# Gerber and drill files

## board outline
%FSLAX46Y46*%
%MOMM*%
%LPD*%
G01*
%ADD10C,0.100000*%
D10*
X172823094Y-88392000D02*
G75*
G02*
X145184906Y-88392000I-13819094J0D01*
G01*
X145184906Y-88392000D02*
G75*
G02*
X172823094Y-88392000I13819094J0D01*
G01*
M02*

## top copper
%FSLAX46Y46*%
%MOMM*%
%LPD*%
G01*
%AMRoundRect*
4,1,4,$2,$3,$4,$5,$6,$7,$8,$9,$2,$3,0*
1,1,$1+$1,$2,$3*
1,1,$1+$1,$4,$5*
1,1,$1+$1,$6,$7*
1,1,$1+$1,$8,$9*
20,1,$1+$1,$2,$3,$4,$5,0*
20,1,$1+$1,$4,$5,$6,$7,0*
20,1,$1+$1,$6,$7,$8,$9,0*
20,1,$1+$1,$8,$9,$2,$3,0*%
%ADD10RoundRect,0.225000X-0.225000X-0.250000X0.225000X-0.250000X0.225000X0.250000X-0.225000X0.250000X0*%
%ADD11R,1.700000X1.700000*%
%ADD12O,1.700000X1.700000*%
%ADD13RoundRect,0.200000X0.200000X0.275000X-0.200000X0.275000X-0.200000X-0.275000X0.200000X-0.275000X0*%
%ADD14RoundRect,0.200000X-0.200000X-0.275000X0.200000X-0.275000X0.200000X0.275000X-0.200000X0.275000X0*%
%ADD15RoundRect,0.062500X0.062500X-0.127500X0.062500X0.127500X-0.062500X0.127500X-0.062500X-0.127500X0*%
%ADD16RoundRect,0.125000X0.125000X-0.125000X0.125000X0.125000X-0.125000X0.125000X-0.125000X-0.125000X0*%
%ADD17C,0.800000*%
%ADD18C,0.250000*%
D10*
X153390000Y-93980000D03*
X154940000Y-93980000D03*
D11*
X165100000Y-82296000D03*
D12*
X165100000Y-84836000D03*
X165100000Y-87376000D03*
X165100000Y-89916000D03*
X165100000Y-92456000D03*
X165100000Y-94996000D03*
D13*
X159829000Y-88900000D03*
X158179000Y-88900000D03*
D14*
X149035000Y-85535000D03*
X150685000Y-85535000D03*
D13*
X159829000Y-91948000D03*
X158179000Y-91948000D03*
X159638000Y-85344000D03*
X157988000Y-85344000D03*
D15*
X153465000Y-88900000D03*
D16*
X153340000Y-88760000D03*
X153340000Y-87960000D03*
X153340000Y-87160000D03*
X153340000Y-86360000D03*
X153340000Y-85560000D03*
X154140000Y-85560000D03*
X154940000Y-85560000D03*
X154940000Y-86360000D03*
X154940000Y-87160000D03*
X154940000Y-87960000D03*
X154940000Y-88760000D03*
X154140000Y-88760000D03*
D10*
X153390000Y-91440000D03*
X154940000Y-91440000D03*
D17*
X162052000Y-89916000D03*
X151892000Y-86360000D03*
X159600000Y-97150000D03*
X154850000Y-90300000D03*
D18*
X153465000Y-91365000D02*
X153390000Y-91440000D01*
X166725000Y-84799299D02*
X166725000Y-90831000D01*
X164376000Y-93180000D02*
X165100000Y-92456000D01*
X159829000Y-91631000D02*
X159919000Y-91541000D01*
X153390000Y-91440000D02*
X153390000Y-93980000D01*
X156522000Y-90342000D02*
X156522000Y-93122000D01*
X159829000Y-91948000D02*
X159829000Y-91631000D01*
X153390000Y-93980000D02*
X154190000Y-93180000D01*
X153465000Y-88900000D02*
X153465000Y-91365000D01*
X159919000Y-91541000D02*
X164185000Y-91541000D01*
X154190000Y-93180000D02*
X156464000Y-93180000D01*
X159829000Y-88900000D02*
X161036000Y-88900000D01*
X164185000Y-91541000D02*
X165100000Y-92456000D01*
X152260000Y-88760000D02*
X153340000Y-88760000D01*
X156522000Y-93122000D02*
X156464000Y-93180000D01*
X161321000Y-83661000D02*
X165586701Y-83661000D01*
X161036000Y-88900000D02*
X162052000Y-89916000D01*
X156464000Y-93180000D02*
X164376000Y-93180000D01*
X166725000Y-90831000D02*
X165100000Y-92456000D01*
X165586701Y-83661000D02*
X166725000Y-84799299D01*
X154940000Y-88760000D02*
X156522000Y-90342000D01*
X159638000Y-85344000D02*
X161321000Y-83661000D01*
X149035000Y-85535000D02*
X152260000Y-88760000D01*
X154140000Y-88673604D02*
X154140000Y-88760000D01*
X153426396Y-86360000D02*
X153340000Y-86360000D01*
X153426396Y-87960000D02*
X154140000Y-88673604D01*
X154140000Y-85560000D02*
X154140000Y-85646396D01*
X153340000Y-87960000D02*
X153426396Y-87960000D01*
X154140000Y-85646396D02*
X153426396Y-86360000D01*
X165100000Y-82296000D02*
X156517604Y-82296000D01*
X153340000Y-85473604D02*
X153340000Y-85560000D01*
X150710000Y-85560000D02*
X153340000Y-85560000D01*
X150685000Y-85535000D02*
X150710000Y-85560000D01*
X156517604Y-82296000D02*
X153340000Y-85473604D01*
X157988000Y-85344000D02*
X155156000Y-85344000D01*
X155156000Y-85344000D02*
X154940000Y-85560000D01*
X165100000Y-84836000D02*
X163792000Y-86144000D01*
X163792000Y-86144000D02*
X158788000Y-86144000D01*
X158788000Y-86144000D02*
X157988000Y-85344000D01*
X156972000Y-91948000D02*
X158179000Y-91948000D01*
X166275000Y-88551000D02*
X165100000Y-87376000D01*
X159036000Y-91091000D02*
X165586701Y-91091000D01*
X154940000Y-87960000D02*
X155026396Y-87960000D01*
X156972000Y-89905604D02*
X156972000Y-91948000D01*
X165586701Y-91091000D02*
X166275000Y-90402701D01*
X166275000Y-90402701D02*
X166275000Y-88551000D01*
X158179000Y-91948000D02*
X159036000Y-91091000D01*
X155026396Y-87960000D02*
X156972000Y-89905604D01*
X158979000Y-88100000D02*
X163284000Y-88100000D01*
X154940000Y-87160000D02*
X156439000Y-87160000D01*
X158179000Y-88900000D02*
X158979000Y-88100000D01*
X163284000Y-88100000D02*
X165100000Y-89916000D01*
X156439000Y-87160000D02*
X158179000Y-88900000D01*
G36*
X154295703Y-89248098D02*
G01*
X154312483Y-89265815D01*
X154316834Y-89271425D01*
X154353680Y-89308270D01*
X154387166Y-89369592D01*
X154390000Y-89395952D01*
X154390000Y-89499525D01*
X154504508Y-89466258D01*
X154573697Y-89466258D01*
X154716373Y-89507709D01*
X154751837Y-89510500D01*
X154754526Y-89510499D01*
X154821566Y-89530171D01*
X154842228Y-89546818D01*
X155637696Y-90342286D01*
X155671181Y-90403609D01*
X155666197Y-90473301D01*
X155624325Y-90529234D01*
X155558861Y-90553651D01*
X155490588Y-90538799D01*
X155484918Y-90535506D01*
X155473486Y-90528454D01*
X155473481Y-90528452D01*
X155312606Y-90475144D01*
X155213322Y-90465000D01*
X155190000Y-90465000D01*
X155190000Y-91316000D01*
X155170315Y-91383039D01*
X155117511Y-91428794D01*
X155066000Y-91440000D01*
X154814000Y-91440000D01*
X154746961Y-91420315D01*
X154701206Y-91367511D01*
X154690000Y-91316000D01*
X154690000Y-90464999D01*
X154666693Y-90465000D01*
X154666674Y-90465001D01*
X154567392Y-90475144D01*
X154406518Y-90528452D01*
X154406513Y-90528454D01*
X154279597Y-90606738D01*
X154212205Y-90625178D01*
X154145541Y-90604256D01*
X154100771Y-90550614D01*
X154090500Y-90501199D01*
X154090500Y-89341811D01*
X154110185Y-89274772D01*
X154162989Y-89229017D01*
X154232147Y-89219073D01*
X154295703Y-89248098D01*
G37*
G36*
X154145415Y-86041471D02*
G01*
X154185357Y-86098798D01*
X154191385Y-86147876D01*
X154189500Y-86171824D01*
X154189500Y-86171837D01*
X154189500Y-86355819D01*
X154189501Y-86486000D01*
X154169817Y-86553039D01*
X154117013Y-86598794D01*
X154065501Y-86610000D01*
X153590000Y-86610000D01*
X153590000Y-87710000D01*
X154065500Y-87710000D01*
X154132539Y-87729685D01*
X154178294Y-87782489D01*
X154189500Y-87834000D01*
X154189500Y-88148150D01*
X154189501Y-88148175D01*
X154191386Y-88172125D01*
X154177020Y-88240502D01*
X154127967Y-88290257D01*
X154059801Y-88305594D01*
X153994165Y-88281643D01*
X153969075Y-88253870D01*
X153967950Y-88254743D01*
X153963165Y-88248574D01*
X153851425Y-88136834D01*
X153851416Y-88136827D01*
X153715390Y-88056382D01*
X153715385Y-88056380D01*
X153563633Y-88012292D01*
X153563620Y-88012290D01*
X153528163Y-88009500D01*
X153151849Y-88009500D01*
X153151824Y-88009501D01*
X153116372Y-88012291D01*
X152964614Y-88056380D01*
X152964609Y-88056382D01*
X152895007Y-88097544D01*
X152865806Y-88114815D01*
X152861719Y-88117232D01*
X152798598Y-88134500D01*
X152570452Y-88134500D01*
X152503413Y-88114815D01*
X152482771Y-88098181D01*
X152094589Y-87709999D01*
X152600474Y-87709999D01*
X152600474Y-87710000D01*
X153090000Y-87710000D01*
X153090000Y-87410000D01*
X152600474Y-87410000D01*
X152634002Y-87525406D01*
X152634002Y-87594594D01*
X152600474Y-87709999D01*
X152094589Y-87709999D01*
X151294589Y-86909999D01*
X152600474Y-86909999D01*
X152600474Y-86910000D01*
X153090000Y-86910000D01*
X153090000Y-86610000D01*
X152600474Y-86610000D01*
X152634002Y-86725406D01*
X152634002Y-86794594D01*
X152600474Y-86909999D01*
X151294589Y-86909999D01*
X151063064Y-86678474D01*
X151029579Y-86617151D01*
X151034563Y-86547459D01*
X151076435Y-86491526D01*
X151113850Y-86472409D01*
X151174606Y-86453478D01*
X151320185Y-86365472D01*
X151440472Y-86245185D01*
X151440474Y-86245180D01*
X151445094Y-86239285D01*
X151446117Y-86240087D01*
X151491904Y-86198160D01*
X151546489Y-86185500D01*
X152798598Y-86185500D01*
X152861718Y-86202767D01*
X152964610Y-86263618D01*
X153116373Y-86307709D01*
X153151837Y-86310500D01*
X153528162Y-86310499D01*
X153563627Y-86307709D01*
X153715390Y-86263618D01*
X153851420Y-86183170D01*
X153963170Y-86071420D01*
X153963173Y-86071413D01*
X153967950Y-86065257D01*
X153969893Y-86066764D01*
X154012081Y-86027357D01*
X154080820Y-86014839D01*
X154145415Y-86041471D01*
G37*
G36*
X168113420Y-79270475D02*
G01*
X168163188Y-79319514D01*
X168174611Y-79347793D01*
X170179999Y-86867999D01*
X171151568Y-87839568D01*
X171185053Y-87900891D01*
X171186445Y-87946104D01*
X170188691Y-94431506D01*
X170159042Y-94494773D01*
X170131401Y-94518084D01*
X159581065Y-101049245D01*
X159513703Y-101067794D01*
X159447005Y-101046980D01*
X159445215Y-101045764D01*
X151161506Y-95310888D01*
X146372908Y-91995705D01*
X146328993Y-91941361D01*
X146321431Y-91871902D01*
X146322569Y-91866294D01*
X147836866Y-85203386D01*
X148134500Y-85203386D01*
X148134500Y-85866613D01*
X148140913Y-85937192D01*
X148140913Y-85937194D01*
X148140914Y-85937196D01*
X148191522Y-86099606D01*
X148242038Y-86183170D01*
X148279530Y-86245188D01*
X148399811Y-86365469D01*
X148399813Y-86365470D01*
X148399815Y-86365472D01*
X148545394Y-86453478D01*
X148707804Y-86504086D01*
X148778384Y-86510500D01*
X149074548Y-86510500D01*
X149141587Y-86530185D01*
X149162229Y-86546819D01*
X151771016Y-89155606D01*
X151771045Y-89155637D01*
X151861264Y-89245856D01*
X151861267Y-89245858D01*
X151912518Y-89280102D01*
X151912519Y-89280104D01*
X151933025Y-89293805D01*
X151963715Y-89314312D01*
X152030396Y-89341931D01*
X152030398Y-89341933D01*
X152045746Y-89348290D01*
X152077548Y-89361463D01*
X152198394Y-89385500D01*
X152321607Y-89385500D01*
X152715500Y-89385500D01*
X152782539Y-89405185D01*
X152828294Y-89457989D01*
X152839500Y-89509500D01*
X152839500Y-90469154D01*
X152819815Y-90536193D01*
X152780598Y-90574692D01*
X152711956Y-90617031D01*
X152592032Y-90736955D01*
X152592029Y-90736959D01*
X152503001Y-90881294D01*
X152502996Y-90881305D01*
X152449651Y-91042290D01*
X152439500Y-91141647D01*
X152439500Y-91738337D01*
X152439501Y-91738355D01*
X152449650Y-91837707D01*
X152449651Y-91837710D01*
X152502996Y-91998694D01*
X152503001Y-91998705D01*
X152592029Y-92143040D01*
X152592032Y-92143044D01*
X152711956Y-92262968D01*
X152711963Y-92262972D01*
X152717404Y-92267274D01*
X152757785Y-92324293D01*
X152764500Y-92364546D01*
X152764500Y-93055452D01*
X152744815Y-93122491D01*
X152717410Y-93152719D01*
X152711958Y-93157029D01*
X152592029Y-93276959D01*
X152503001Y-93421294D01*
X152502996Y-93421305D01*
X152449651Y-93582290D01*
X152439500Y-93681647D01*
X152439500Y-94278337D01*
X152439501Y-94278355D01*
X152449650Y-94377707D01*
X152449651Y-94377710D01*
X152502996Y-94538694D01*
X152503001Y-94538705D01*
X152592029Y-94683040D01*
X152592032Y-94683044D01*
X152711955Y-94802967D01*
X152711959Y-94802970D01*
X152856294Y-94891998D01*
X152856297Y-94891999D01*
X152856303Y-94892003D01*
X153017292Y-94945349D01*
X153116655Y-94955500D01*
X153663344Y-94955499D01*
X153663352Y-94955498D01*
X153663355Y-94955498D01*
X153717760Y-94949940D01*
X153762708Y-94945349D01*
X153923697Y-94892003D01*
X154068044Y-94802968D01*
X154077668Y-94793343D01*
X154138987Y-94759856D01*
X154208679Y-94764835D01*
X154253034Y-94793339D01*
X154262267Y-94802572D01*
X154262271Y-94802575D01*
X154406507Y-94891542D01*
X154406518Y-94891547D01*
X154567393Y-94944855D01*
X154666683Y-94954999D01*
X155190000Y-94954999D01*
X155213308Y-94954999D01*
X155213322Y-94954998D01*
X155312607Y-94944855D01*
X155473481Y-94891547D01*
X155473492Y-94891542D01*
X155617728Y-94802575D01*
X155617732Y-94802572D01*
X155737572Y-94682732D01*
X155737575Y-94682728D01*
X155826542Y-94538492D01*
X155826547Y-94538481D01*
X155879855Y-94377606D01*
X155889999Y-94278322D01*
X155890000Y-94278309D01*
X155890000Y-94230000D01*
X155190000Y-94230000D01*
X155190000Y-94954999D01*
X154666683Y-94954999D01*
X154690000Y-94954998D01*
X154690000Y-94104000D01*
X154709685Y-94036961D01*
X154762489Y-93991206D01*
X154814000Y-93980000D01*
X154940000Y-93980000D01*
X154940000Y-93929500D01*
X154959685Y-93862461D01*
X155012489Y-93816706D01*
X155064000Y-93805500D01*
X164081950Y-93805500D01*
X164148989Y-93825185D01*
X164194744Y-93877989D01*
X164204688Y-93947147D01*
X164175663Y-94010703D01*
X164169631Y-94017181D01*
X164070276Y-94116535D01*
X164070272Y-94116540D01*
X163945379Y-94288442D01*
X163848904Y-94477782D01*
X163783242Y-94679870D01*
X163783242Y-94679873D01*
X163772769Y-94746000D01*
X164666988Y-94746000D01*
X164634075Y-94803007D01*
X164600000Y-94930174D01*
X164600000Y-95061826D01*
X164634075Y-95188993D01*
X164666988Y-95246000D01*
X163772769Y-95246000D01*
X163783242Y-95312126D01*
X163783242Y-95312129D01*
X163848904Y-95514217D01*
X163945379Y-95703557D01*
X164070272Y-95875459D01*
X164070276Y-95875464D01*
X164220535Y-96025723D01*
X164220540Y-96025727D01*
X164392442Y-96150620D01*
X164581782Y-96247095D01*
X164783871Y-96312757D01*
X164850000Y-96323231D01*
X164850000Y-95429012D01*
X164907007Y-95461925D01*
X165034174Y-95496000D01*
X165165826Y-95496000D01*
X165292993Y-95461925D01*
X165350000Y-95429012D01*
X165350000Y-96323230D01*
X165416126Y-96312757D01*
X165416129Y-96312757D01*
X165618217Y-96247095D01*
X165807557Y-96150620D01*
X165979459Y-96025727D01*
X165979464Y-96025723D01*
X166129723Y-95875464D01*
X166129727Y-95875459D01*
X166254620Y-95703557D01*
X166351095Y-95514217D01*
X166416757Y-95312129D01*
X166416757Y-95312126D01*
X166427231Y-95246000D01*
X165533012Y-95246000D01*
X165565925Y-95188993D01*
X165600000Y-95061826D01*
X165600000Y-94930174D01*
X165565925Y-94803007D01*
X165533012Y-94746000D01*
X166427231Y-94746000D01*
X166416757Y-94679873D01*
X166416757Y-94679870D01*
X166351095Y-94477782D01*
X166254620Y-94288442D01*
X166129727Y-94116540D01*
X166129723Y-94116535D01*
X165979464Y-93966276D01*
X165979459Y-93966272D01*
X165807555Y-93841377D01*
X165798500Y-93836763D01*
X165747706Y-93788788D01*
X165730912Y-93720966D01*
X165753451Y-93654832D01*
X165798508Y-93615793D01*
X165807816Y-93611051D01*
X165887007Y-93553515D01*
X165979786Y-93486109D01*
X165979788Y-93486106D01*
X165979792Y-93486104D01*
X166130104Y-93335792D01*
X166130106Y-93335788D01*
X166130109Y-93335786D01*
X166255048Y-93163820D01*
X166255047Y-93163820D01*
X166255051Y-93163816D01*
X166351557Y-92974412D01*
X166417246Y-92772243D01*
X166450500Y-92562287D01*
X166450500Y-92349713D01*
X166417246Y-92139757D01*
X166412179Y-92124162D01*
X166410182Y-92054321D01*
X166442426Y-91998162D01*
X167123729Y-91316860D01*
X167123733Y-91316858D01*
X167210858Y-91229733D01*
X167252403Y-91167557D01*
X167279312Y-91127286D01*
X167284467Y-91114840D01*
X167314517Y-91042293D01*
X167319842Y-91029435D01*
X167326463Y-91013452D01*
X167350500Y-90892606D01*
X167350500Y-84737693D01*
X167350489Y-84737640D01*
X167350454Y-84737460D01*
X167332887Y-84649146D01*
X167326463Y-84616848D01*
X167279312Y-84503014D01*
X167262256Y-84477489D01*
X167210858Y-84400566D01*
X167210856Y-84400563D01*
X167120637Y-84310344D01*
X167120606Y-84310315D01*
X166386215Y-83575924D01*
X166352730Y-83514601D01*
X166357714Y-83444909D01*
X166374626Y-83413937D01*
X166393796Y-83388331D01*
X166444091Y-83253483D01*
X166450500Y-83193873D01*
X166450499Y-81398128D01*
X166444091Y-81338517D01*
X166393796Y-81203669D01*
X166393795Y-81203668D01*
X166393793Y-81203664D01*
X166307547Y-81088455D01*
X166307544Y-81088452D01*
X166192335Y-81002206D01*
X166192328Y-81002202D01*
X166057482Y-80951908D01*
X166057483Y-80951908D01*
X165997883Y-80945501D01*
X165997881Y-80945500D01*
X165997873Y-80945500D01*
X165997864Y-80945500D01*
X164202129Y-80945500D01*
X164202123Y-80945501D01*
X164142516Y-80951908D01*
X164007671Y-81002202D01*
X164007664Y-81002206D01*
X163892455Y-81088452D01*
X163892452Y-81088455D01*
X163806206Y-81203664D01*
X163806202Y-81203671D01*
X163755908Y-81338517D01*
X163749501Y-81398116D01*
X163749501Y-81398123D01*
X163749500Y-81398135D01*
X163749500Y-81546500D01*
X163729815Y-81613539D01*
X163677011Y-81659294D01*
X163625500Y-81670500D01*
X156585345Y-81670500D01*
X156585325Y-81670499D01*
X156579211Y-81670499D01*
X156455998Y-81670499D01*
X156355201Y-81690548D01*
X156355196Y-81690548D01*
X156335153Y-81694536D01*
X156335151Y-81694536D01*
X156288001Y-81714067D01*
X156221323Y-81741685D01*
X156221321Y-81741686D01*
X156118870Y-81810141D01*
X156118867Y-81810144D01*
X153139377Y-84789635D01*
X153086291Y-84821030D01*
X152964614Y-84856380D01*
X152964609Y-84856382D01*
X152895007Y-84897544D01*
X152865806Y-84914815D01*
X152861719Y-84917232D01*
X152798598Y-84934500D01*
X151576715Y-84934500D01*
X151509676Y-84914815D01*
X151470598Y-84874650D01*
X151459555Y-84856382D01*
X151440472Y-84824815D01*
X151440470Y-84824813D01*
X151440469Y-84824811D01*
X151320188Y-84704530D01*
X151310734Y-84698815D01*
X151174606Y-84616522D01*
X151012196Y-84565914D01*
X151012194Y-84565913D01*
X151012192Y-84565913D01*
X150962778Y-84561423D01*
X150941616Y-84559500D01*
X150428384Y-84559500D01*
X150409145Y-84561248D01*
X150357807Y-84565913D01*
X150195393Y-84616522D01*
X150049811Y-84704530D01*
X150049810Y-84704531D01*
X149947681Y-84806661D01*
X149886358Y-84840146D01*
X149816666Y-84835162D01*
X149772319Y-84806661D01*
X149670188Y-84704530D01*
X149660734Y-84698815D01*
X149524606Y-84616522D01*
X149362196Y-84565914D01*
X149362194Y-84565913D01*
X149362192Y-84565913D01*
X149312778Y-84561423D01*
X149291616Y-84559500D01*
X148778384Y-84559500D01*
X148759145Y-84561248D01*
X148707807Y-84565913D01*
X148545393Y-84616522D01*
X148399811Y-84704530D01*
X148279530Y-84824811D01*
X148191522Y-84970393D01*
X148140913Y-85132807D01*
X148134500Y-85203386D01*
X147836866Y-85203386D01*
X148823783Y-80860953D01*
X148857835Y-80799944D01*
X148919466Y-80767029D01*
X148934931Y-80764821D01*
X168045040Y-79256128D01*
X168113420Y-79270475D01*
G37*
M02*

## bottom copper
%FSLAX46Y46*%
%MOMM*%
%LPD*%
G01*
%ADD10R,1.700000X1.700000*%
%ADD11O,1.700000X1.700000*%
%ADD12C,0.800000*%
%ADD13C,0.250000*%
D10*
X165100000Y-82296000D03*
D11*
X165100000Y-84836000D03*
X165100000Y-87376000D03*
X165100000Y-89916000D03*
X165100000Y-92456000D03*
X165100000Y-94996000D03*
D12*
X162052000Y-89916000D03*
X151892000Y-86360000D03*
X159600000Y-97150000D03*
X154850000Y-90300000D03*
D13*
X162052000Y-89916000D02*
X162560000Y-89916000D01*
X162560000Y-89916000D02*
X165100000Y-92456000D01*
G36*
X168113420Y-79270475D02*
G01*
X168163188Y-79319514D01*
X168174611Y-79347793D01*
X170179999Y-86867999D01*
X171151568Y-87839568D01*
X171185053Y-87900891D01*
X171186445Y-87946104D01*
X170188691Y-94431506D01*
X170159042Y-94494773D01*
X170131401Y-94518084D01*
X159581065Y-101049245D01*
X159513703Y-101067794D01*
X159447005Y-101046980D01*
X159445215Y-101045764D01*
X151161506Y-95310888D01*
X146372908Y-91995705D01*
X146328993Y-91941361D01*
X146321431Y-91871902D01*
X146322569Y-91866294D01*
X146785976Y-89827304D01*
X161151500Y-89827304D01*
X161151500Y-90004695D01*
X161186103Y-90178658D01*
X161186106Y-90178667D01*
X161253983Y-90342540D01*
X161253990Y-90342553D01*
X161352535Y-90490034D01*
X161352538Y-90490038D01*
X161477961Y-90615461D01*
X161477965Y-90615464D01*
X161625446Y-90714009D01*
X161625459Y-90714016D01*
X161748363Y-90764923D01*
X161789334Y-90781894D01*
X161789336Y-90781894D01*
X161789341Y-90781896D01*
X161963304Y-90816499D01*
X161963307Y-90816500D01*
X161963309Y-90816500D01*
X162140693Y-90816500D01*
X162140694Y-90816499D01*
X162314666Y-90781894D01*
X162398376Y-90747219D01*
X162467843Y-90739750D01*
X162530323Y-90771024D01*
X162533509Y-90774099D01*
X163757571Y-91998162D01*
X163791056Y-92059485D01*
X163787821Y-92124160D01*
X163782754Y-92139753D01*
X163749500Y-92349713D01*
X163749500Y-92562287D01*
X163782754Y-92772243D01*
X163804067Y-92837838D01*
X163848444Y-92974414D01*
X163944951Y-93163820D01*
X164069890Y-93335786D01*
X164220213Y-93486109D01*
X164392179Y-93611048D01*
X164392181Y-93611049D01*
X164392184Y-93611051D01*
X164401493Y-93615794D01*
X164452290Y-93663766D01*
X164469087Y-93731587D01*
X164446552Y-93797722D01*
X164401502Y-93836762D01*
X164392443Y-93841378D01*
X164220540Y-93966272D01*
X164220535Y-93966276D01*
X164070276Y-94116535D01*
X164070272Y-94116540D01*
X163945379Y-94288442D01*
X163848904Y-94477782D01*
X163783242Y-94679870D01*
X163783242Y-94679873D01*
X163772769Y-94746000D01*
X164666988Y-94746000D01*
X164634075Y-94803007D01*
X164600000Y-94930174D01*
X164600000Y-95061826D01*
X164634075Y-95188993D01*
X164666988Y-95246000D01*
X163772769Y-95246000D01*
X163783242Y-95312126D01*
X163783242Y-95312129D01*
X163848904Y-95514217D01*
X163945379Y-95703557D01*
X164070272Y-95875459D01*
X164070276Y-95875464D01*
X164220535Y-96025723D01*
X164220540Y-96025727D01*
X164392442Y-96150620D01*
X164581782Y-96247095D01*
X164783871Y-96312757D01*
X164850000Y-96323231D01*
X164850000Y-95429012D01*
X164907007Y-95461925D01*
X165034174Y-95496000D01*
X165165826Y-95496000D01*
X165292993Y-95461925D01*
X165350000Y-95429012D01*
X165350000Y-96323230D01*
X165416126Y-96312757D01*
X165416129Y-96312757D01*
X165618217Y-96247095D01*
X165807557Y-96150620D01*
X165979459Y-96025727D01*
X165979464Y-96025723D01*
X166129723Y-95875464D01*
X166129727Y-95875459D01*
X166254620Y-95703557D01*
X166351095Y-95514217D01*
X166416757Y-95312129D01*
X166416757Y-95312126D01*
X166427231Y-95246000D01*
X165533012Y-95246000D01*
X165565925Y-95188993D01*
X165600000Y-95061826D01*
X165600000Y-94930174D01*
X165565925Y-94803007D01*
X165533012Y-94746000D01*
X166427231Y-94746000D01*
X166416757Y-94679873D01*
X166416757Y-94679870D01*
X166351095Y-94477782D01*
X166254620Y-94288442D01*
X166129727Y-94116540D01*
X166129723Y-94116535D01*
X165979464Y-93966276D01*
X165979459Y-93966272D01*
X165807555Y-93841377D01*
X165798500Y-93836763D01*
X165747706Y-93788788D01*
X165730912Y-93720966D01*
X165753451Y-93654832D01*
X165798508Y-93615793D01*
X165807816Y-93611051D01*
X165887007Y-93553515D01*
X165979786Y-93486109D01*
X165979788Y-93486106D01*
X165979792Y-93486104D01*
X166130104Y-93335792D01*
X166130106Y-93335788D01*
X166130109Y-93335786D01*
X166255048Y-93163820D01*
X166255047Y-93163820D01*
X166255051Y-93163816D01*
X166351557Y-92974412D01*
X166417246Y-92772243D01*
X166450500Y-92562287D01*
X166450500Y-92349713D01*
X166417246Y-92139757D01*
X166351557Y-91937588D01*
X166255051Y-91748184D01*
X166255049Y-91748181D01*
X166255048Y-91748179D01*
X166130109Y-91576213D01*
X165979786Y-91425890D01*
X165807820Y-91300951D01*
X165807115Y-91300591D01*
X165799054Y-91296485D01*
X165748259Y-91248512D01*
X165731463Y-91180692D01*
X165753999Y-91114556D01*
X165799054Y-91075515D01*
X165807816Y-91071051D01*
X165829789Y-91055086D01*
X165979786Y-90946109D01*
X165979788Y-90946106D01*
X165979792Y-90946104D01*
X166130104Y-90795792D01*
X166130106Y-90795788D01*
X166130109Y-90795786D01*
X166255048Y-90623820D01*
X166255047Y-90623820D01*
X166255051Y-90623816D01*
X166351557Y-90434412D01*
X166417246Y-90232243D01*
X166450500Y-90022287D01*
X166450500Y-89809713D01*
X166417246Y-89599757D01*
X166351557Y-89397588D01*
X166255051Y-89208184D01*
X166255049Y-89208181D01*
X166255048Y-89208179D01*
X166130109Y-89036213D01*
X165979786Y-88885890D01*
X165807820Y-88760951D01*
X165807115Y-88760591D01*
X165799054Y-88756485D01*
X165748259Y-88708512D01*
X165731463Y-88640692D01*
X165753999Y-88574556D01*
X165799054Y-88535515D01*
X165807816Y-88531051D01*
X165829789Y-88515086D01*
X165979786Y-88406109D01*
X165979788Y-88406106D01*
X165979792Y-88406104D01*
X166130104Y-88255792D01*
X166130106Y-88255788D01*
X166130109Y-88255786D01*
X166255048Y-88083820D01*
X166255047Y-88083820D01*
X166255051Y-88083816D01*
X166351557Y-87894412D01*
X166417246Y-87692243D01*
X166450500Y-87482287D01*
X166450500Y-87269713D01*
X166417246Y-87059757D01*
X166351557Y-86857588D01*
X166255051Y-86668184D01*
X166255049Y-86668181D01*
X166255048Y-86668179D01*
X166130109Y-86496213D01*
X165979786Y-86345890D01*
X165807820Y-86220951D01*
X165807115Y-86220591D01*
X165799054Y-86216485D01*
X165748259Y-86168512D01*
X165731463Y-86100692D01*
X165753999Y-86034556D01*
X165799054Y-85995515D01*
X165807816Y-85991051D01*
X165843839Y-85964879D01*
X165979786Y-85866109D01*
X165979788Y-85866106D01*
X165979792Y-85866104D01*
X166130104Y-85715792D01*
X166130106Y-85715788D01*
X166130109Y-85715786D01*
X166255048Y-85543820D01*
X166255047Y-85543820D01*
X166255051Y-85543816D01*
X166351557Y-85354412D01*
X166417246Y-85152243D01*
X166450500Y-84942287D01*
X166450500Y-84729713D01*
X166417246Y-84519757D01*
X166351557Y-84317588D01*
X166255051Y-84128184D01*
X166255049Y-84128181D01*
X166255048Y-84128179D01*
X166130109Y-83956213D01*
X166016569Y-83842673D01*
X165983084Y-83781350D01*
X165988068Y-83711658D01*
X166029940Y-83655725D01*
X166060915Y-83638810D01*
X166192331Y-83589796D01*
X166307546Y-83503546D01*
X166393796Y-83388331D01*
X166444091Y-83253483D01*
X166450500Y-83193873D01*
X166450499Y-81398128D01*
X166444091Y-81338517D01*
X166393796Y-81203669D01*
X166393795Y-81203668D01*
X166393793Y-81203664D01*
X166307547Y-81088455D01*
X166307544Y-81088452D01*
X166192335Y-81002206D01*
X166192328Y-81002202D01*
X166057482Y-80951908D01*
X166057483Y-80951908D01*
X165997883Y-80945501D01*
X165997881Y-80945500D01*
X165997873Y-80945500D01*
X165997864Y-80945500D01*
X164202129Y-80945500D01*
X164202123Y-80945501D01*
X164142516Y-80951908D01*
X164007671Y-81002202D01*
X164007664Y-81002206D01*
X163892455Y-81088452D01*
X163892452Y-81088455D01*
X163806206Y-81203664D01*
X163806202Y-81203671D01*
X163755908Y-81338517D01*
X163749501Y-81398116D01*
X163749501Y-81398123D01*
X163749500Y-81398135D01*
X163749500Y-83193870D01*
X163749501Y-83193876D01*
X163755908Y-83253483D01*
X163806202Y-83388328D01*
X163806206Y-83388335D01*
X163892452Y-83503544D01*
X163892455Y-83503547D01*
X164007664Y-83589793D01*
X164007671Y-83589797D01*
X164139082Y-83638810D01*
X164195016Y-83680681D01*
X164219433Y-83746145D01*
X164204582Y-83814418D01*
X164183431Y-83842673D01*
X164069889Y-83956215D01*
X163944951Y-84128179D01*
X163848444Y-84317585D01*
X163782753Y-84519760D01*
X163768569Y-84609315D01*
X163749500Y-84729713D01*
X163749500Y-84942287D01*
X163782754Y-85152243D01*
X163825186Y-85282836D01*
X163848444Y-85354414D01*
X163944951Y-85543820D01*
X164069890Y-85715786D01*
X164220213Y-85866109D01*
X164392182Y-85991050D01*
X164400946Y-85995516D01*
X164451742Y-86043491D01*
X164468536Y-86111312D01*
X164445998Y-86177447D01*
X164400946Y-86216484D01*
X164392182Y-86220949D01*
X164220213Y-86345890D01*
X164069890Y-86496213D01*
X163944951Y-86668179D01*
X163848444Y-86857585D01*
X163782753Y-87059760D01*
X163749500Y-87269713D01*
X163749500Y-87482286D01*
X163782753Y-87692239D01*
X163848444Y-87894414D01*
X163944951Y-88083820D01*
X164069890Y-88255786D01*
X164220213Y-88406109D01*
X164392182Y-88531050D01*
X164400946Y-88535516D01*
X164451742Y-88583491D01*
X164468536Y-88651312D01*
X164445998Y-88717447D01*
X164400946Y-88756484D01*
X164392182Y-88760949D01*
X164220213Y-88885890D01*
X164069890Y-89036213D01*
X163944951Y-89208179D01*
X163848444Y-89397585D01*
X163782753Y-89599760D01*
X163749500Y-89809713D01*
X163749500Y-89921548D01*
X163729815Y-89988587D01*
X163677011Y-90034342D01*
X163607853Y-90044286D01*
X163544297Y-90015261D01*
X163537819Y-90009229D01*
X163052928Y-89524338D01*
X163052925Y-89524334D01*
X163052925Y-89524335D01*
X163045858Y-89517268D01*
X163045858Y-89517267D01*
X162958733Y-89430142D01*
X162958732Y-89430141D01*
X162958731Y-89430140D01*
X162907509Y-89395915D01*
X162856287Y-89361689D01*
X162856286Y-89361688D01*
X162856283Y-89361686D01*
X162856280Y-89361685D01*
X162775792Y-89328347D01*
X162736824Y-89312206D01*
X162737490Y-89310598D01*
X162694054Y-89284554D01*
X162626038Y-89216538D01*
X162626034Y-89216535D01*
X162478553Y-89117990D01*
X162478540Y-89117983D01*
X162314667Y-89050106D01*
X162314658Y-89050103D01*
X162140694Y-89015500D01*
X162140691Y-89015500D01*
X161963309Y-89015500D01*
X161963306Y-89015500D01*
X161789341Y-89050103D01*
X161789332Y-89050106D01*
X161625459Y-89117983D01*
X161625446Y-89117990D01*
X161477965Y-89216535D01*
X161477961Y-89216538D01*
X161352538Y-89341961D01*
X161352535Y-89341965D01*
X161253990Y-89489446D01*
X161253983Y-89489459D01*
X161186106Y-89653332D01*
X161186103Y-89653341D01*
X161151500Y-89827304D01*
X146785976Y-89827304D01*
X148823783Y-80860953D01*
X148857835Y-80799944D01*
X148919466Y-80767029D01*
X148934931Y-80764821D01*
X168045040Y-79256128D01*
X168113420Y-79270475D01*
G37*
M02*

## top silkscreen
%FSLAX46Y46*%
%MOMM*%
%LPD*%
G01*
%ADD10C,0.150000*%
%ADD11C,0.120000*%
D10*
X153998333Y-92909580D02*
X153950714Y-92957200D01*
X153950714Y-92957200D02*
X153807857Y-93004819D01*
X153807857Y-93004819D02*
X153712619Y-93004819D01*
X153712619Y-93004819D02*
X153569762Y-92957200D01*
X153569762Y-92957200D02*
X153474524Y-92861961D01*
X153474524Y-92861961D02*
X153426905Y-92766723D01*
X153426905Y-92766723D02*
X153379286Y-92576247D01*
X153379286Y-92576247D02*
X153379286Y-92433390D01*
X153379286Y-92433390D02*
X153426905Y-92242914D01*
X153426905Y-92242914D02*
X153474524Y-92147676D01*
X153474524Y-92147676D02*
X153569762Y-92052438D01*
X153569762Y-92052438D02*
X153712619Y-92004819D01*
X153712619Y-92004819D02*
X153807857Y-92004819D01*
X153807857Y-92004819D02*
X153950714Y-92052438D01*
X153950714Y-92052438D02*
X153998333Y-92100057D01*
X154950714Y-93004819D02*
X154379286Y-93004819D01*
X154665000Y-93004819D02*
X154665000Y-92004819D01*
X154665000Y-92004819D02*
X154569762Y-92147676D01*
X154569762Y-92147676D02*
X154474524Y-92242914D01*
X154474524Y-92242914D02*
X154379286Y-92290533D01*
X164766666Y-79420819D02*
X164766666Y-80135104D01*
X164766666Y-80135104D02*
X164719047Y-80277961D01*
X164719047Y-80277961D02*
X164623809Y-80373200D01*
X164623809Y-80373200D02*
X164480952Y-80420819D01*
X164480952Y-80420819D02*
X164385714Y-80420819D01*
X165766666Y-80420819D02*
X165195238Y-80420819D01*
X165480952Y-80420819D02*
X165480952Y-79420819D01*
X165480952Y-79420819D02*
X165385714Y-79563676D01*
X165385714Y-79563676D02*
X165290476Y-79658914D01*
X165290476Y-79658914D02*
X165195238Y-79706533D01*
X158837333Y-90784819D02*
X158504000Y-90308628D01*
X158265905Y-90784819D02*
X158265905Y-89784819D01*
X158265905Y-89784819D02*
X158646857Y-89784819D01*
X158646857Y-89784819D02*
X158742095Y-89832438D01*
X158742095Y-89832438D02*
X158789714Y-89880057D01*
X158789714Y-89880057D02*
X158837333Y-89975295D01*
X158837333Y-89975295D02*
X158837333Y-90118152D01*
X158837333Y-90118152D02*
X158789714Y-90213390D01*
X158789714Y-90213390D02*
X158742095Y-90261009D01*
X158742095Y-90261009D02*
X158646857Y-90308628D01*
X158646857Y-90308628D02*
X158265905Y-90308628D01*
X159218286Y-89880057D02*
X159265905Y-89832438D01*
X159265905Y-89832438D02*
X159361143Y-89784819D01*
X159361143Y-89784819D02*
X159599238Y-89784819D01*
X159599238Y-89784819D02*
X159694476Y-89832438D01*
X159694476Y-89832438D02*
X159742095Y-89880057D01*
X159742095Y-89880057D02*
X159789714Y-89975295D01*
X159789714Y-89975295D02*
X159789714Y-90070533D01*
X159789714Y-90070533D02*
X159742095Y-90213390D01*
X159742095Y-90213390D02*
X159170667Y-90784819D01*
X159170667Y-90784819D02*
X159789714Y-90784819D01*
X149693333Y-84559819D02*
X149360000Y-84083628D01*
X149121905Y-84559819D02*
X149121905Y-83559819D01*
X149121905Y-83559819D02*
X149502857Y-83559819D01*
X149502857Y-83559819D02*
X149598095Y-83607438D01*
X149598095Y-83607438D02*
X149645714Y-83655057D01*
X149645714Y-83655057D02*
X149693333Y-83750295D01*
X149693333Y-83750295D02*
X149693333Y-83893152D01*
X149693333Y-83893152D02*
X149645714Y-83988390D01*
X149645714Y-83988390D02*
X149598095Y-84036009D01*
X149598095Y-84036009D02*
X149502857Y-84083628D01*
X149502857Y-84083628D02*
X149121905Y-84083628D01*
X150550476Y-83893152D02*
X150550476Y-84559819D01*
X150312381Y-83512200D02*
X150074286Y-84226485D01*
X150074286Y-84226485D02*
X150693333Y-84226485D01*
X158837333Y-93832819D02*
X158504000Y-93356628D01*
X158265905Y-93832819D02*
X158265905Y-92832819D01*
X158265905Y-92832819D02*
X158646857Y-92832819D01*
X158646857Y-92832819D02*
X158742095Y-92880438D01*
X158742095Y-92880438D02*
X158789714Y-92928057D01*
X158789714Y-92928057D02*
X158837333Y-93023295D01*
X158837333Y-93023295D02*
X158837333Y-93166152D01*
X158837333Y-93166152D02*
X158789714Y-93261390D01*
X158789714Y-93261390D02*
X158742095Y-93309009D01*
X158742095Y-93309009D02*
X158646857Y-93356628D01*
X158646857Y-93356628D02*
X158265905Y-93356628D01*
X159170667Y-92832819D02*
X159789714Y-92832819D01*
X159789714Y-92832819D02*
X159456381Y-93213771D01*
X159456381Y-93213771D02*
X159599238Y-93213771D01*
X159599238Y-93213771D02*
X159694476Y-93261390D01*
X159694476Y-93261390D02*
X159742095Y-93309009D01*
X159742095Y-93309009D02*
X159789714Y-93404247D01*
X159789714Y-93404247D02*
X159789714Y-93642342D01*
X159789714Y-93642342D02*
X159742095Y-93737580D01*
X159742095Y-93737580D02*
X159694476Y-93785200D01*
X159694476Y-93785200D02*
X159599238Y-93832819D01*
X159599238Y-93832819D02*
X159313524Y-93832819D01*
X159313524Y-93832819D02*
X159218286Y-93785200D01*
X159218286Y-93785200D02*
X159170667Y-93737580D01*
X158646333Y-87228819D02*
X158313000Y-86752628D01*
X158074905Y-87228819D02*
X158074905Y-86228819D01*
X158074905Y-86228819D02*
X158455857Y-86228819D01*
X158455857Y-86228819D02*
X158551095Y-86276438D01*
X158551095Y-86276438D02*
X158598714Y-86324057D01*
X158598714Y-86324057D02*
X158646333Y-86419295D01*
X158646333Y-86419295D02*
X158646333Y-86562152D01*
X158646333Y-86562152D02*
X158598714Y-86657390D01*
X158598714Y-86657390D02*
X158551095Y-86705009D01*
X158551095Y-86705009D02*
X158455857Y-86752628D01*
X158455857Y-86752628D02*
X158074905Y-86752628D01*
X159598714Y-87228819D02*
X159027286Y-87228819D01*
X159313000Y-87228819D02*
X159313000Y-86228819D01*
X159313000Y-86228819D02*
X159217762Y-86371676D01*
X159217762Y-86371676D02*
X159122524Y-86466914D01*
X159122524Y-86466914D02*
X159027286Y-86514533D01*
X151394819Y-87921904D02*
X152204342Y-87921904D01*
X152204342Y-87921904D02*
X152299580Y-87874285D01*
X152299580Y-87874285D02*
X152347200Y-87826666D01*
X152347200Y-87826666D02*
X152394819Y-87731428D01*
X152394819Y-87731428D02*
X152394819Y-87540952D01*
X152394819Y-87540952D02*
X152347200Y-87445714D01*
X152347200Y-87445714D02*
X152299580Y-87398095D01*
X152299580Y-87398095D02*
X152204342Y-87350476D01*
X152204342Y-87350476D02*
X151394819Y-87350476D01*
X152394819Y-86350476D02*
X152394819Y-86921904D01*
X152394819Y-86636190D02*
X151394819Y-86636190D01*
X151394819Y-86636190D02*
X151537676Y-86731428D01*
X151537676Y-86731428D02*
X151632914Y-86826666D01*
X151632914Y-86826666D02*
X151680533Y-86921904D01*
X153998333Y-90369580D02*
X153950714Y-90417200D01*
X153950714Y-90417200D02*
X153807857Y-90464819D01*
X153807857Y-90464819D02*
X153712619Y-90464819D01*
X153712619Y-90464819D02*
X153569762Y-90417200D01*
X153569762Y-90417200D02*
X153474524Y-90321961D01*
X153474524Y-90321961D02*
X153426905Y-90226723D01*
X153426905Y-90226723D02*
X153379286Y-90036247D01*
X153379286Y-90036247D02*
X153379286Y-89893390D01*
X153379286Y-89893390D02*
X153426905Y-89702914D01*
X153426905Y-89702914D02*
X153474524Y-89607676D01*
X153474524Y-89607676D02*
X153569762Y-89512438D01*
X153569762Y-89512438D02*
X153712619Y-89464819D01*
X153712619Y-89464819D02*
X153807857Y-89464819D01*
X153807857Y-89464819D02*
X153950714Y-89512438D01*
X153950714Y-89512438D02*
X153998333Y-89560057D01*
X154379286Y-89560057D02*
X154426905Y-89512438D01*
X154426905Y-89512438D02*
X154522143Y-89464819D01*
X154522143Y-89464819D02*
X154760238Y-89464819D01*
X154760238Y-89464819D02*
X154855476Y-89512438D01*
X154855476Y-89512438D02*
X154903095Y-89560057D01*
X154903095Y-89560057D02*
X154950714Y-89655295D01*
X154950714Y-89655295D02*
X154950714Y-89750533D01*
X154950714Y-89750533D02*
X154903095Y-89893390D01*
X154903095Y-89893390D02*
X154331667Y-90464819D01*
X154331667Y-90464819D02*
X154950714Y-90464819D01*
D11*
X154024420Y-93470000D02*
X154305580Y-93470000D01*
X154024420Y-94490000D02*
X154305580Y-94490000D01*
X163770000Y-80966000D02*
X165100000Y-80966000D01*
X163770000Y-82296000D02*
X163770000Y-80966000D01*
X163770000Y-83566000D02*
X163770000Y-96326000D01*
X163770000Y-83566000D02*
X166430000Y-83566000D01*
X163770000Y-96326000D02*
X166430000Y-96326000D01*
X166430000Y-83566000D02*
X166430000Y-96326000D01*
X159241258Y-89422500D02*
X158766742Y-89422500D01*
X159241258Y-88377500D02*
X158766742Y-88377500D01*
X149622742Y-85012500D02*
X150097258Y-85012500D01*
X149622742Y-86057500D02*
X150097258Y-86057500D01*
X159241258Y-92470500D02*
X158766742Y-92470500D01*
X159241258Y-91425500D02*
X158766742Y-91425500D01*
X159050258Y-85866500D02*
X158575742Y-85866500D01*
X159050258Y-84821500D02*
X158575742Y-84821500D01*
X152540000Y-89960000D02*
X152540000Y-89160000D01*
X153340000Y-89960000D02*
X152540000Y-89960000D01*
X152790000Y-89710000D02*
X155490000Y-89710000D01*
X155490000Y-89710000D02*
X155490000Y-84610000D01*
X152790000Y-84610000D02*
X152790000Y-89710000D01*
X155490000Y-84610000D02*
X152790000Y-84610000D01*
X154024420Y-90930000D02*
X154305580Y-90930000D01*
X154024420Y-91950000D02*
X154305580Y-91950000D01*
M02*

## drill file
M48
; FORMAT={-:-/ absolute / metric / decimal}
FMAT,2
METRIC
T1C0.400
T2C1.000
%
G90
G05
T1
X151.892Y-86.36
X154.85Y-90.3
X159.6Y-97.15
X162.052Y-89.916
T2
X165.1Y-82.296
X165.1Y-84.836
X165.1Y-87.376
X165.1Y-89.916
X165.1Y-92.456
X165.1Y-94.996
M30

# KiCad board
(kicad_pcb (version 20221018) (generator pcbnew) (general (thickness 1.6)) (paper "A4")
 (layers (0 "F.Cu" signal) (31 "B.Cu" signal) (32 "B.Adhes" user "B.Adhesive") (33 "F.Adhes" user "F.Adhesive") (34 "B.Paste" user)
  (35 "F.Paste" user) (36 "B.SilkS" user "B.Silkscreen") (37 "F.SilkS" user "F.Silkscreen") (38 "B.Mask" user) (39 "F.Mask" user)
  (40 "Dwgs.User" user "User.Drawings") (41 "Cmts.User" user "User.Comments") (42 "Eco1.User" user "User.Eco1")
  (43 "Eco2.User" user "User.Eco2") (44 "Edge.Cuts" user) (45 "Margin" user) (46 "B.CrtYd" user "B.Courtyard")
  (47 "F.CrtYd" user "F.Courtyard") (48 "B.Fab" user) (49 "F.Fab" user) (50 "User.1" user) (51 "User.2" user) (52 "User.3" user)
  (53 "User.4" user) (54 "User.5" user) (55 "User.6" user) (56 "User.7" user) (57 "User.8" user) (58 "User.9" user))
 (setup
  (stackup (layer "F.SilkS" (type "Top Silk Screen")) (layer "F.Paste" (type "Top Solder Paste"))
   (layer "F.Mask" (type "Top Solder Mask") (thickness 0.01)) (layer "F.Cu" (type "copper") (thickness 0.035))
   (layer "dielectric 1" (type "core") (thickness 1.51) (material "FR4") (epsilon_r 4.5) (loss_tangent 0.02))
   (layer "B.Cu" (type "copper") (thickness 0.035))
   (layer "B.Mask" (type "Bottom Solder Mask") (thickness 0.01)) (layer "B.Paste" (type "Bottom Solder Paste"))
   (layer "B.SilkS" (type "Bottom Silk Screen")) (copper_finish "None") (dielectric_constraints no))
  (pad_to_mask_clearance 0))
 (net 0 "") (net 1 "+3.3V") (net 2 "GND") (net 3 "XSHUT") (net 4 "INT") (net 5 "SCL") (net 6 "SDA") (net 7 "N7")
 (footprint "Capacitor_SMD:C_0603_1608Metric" (layer "F.Cu") (at 154.165 93.98)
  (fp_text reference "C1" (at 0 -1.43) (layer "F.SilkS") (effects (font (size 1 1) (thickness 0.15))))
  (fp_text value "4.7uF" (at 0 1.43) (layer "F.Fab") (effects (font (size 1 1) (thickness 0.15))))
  (fp_line (start -0.14058 -0.51) (end 0.14058 -0.51) (stroke (width 0.12) (type solid)) (layer "F.SilkS"))
  (fp_line (start -0.14058 0.51) (end 0.14058 0.51) (stroke (width 0.12) (type solid)) (layer "F.SilkS"))
  (pad "1" smd roundrect (at -0.775 0) (size 0.9 0.95) (layers "F.Cu" "F.Paste" "F.Mask") (roundrect_rratio 0.25) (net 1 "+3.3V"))
  (pad "2" smd roundrect (at 0.775 0) (size 0.9 0.95) (layers "F.Cu" "F.Paste" "F.Mask") (roundrect_rratio 0.25) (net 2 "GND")))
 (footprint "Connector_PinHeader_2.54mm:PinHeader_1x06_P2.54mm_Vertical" (layer "F.Cu") (at 165.1 82.296)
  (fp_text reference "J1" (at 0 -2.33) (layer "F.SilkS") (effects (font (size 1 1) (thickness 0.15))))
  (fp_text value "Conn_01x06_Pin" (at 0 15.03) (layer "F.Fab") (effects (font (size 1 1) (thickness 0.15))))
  (fp_line (start -1.33 -1.33) (end 0 -1.33) (stroke (width 0.12) (type solid)) (layer "F.SilkS"))
  (fp_line (start -1.33 0) (end -1.33 -1.33) (stroke (width 0.12) (type solid)) (layer "F.SilkS"))
  (fp_line (start -1.33 1.27) (end -1.33 14.03) (stroke (width 0.12) (type solid)) (layer "F.SilkS"))
  (fp_line (start -1.33 1.27) (end 1.33 1.27) (stroke (width 0.12) (type solid)) (layer "F.SilkS"))
  (fp_line (start -1.33 14.03) (end 1.33 14.03) (stroke (width 0.12) (type solid)) (layer "F.SilkS"))
  (fp_line (start 1.33 1.27) (end 1.33 14.03) (stroke (width 0.12) (type solid)) (layer "F.SilkS"))
  (pad "1" thru_hole rect (at 0 0) (size 1.7 1.7) (drill 1) (layers "*.Cu" "*.Mask") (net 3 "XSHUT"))
  (pad "2" thru_hole oval (at 0 2.54) (size 1.7 1.7) (drill 1) (layers "*.Cu" "*.Mask") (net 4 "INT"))
  (pad "3" thru_hole oval (at 0 5.08) (size 1.7 1.7) (drill 1) (layers "*.Cu" "*.Mask") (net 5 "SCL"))
  (pad "4" thru_hole oval (at 0 7.62) (size 1.7 1.7) (drill 1) (layers "*.Cu" "*.Mask") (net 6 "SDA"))
  (pad "5" thru_hole oval (at 0 10.16) (size 1.7 1.7) (drill 1) (layers "*.Cu" "*.Mask") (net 1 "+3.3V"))
  (pad "6" thru_hole oval (at 0 12.7) (size 1.7 1.7) (drill 1) (layers "*.Cu" "*.Mask") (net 2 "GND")))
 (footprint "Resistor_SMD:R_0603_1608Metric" (layer "F.Cu") (at 159.004 88.9 180)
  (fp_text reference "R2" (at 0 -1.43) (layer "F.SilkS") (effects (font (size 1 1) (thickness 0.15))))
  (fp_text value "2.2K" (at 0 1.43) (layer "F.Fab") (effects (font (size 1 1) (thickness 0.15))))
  (fp_line (start -0.237258 -0.5225) (end 0.237258 -0.5225) (stroke (width 0.12) (type solid)) (layer "F.SilkS"))
  (fp_line (start -0.237258 0.5225) (end 0.237258 0.5225) (stroke (width 0.12) (type solid)) (layer "F.SilkS"))
  (pad "1" smd roundrect (at -0.825 0 180) (size 0.8 0.95) (layers "F.Cu" "F.Paste" "F.Mask") (roundrect_rratio 0.25) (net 1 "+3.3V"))
  (pad "2" smd roundrect (at 0.825 0 180) (size 0.8 0.95) (layers "F.Cu" "F.Paste" "F.Mask") (roundrect_rratio 0.25) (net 6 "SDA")))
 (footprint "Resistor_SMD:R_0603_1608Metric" (layer "F.Cu") (at 149.86 85.535)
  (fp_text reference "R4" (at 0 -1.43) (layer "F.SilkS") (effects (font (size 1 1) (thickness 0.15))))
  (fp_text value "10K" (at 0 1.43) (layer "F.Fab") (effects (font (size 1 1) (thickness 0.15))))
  (fp_line (start -0.237258 -0.5225) (end 0.237258 -0.5225) (stroke (width 0.12) (type solid)) (layer "F.SilkS"))
  (fp_line (start -0.237258 0.5225) (end 0.237258 0.5225) (stroke (width 0.12) (type solid)) (layer "F.SilkS"))
  (pad "1" smd roundrect (at -0.825 0) (size 0.8 0.95) (layers "F.Cu" "F.Paste" "F.Mask") (roundrect_rratio 0.25) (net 1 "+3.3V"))
  (pad "2" smd roundrect (at 0.825 0) (size 0.8 0.95) (layers "F.Cu" "F.Paste" "F.Mask") (roundrect_rratio 0.25) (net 3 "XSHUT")))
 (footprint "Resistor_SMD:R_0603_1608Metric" (layer "F.Cu") (at 159.004 91.948 180)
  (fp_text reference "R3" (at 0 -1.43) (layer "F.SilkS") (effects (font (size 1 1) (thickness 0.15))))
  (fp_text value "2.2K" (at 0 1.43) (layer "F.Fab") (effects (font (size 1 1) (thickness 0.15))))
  (fp_line (start -0.237258 -0.5225) (end 0.237258 -0.5225) (stroke (width 0.12) (type solid)) (layer "F.SilkS"))
  (fp_line (start -0.237258 0.5225) (end 0.237258 0.5225) (stroke (width 0.12) (type solid)) (layer "F.SilkS"))
  (pad "1" smd roundrect (at -0.825 0 180) (size 0.8 0.95) (layers "F.Cu" "F.Paste" "F.Mask") (roundrect_rratio 0.25) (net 1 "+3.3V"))
  (pad "2" smd roundrect (at 0.825 0 180) (size 0.8 0.95) (layers "F.Cu" "F.Paste" "F.Mask") (roundrect_rratio 0.25) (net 5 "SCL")))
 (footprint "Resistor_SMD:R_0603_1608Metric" (layer "F.Cu") (at 158.813 85.344 180)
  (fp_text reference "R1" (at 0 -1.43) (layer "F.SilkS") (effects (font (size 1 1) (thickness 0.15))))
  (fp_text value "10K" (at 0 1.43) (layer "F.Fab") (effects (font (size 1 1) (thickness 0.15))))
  (fp_line (start -0.237258 -0.5225) (end 0.237258 -0.5225) (stroke (width 0.12) (type solid)) (layer "F.SilkS"))
  (fp_line (start -0.237258 0.5225) (end 0.237258 0.5225) (stroke (width 0.12) (type solid)) (layer "F.SilkS"))
  (pad "1" smd roundrect (at -0.825 0 180) (size 0.8 0.95) (layers "F.Cu" "F.Paste" "F.Mask") (roundrect_rratio 0.25) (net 1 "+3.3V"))
  (pad "2" smd roundrect (at 0.825 0 180) (size 0.8 0.95) (layers "F.Cu" "F.Paste" "F.Mask") (roundrect_rratio 0.25) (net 4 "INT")))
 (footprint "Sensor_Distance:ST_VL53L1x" (layer "F.Cu") (at 154.14 87.16 90)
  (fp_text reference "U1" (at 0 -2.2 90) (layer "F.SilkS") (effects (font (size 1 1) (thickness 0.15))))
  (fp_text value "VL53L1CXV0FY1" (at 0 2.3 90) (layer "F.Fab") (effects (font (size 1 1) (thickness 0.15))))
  (fp_line (start -2.8 -1.6) (end -2 -1.6) (stroke (width 0.12) (type solid)) (layer "F.SilkS"))
  (fp_line (start -2.8 -0.8) (end -2.8 -1.6) (stroke (width 0.12) (type solid)) (layer "F.SilkS"))
  (fp_line (start -2.55 -1.35) (end -2.55 1.35) (stroke (width 0.12) (type solid)) (layer "F.SilkS"))
  (fp_line (start -2.55 1.35) (end 2.55 1.35) (stroke (width 0.12) (type solid)) (layer "F.SilkS"))
  (fp_line (start 2.55 -1.35) (end -2.55 -1.35) (stroke (width 0.12) (type solid)) (layer "F.SilkS"))
  (fp_line (start 2.55 1.35) (end 2.55 -1.35) (stroke (width 0.12) (type solid)) (layer "F.SilkS"))
  (pad "1" smd roundrect (at -1.74 -0.675 90) (size 0.38 0.25) (layers "F.Cu" "F.Paste" "F.Mask") (roundrect_rratio 0.25) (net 1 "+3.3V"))
  (pad "1" smd roundrect (at -1.6 -0.8 90) (size 0.5 0.5) (layers "F.Cu" "F.Paste" "F.Mask") (roundrect_rratio 0.25) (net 1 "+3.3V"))
  (pad "2" smd roundrect (at -0.8 -0.8 90) (size 0.5 0.5) (layers "F.Cu" "F.Paste" "F.Mask") (roundrect_rratio 0.25) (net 2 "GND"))
  (pad "3" smd roundrect (at 0 -0.8 90) (size 0.5 0.5) (layers "F.Cu" "F.Paste" "F.Mask") (roundrect_rratio 0.25) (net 2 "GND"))
  (pad "4" smd roundrect (at 0.8 -0.8 90) (size 0.5 0.5) (layers "F.Cu" "F.Paste" "F.Mask") (roundrect_rratio 0.25) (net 2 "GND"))
  (pad "5" smd roundrect (at 1.6 -0.8 90) (size 0.5 0.5) (layers "F.Cu" "F.Paste" "F.Mask") (roundrect_rratio 0.25) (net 3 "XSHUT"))
  (pad "6" smd roundrect (at 1.6 0 90) (size 0.5 0.5) (layers "F.Cu" "F.Paste" "F.Mask") (roundrect_rratio 0.25) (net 2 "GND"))
  (pad "7" smd roundrect (at 1.6 0.8 90) (size 0.5 0.5) (layers "F.Cu" "F.Paste" "F.Mask") (roundrect_rratio 0.25) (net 4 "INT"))
  (pad "8" smd roundrect (at 0.8 0.8 90) (size 0.5 0.5) (layers "F.Cu" "F.Paste" "F.Mask") (roundrect_rratio 0.25) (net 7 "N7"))
  (pad "9" smd roundrect (at 0 0.8 90) (size 0.5 0.5) (layers "F.Cu" "F.Paste" "F.Mask") (roundrect_rratio 0.25) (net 6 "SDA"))
  (pad "10" smd roundrect (at -0.8 0.8 90) (size 0.5 0.5) (layers "F.Cu" "F.Paste" "F.Mask") (roundrect_rratio 0.25) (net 5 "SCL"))
  (pad "11" smd roundrect (at -1.6 0.8 90) (size 0.5 0.5) (layers "F.Cu" "F.Paste" "F.Mask") (roundrect_rratio 0.25) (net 1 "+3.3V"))
  (pad "12" smd roundrect (at -1.6 0 90) (size 0.5 0.5) (layers "F.Cu" "F.Paste" "F.Mask") (roundrect_rratio 0.25) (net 2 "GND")))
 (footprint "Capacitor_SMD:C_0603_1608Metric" (layer "F.Cu") (at 154.165 91.44)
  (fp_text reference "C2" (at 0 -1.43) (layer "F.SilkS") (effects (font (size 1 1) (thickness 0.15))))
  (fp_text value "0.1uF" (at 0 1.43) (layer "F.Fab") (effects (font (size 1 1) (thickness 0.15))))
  (fp_line (start -0.14058 -0.51) (end 0.14058 -0.51) (stroke (width 0.12) (type solid)) (layer "F.SilkS"))
  (fp_line (start -0.14058 0.51) (end 0.14058 0.51) (stroke (width 0.12) (type solid)) (layer "F.SilkS"))
  (pad "1" smd roundrect (at -0.775 0) (size 0.9 0.95) (layers "F.Cu" "F.Paste" "F.Mask") (roundrect_rratio 0.25) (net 1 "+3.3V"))
  (pad "2" smd roundrect (at 0.775 0) (size 0.9 0.95) (layers "F.Cu" "F.Paste" "F.Mask") (roundrect_rratio 0.25) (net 2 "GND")))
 (gr_circle (center 159.004 88.392) (end 147.828 80.264) (stroke (width 0.1) (type default)) (fill none) (layer "Edge.Cuts"))
 (segment (start 153.465 91.365) (end 153.39 91.44) (width 0.25) (layer "F.Cu") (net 1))
 (segment (start 166.725 84.799299) (end 166.725 90.831) (width 0.25) (layer "F.Cu") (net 1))
 (segment (start 164.376 93.18) (end 165.1 92.456) (width 0.25) (layer "F.Cu") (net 1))
 (segment (start 159.829 91.631) (end 159.919 91.541) (width 0.25) (layer "F.Cu") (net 1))
 (segment (start 153.39 91.44) (end 153.39 93.98) (width 0.25) (layer "F.Cu") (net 1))
 (segment (start 156.522 90.342) (end 156.522 93.122) (width 0.25) (layer "F.Cu") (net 1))
 (segment (start 159.829 91.948) (end 159.829 91.631) (width 0.25) (layer "F.Cu") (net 1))
 (segment (start 153.39 93.98) (end 154.19 93.18) (width 0.25) (layer "F.Cu") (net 1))
 (segment (start 153.465 88.9) (end 153.465 91.365) (width 0.25) (layer "F.Cu") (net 1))
 (segment (start 159.919 91.541) (end 164.185 91.541) (width 0.25) (layer "F.Cu") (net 1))
 (segment (start 154.19 93.18) (end 156.464 93.18) (width 0.25) (layer "F.Cu") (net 1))
 (segment (start 159.829 88.9) (end 161.036 88.9) (width 0.25) (layer "F.Cu") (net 1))
 (segment (start 164.185 91.541) (end 165.1 92.456) (width 0.25) (layer "F.Cu") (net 1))
 (segment (start 152.26 88.76) (end 153.34 88.76) (width 0.25) (layer "F.Cu") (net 1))
 (segment (start 156.522 93.122) (end 156.464 93.18) (width 0.25) (layer "F.Cu") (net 1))
 (segment (start 161.321 83.661) (end 165.586701 83.661) (width 0.25) (layer "F.Cu") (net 1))
 (segment (start 161.036 88.9) (end 162.052 89.916) (width 0.25) (layer "F.Cu") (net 1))
 (segment (start 156.464 93.18) (end 164.376 93.18) (width 0.25) (layer "F.Cu") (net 1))
 (segment (start 166.725 90.831) (end 165.1 92.456) (width 0.25) (layer "F.Cu") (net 1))
 (segment (start 165.586701 83.661) (end 166.725 84.799299) (width 0.25) (layer "F.Cu") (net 1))
 (segment (start 154.94 88.76) (end 156.522 90.342) (width 0.25) (layer "F.Cu") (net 1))
 (segment (start 159.638 85.344) (end 161.321 83.661) (width 0.25) (layer "F.Cu") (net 1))
 (segment (start 149.035 85.535) (end 152.26 88.76) (width 0.25) (layer "F.Cu") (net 1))
 (via (at 162.052 89.916) (size 0.8) (drill 0.4) (layers "F.Cu" "B.Cu") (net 1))
 (segment (start 162.052 89.916) (end 162.56 89.916) (width 0.25) (layer "B.Cu") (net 1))
 (segment (start 162.56 89.916) (end 165.1 92.456) (width 0.25) (layer "B.Cu") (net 1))
 (segment (start 154.14 88.673604) (end 154.14 88.76) (width 0.25) (layer "F.Cu") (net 2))
 (segment (start 153.426396 86.36) (end 153.34 86.36) (width 0.25) (layer "F.Cu") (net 2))
 (segment (start 153.426396 87.96) (end 154.14 88.673604) (width 0.25) (layer "F.Cu") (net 2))
 (segment (start 154.14 85.56) (end 154.14 85.646396) (width 0.25) (layer "F.Cu") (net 2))
 (segment (start 153.34 87.96) (end 153.426396 87.96) (width 0.25) (layer "F.Cu") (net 2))
 (segment (start 154.14 85.646396) (end 153.426396 86.36) (width 0.25) (layer "F.Cu") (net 2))
 (via (at 151.892 86.36) (size 0.8) (drill 0.4) (layers "F.Cu" "B.Cu") (free) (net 2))
 (via (at 159.6 97.15) (size 0.8) (drill 0.4) (layers "F.Cu" "B.Cu") (free) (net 2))
 (via (at 154.85 90.3) (size 0.8) (drill 0.4) (layers "F.Cu" "B.Cu") (free) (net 2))
 (segment (start 165.1 82.296) (end 156.517604 82.296) (width 0.25) (layer "F.Cu") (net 3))
 (segment (start 153.34 85.473604) (end 153.34 85.56) (width 0.25) (layer "F.Cu") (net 3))
 (segment (start 150.71 85.56) (end 153.34 85.56) (width 0.25) (layer "F.Cu") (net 3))
 (segment (start 150.685 85.535) (end 150.71 85.56) (width 0.25) (layer "F.Cu") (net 3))
 (segment (start 156.517604 82.296) (end 153.34 85.473604) (width 0.25) (layer "F.Cu") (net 3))
 (segment (start 157.988 85.344) (end 155.156 85.344) (width 0.25) (layer "F.Cu") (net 4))
 (segment (start 155.156 85.344) (end 154.94 85.56) (width 0.25) (layer "F.Cu") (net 4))
 (segment (start 165.1 84.836) (end 163.792 86.144) (width 0.25) (layer "F.Cu") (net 4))
 (segment (start 163.792 86.144) (end 158.788 86.144) (width 0.25) (layer "F.Cu") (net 4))
 (segment (start 158.788 86.144) (end 157.988 85.344) (width 0.25) (layer "F.Cu") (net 4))
 (segment (start 156.972 91.948) (end 158.179 91.948) (width 0.25) (layer "F.Cu") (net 5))
 (segment (start 166.275 88.551) (end 165.1 87.376) (width 0.25) (layer "F.Cu") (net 5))
 (segment (start 159.036 91.091) (end 165.586701 91.091) (width 0.25) (layer "F.Cu") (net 5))
 (segment (start 154.94 87.96) (end 155.026396 87.96) (width 0.25) (layer "F.Cu") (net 5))
 (segment (start 156.972 89.905604) (end 156.972 91.948) (width 0.25) (layer "F.Cu") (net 5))
 (segment (start 165.586701 91.091) (end 166.275 90.402701) (width 0.25) (layer "F.Cu") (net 5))
 (segment (start 166.275 90.402701) (end 166.275 88.551) (width 0.25) (layer "F.Cu") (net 5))
 (segment (start 158.179 91.948) (end 159.036 91.091) (width 0.25) (layer "F.Cu") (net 5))
 (segment (start 155.026396 87.96) (end 156.972 89.905604) (width 0.25) (layer "F.Cu") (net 5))
 (segment (start 158.979 88.1) (end 163.284 88.1) (width 0.25) (layer "F.Cu") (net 6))
 (segment (start 154.94 87.16) (end 156.439 87.16) (width 0.25) (layer "F.Cu") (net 6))
 (segment (start 158.179 88.9) (end 158.979 88.1) (width 0.25) (layer "F.Cu") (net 6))
 (segment (start 163.284 88.1) (end 165.1 89.916) (width 0.25) (layer "F.Cu") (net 6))
 (segment (start 156.439 87.16) (end 158.179 88.9) (width 0.25) (layer "F.Cu") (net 6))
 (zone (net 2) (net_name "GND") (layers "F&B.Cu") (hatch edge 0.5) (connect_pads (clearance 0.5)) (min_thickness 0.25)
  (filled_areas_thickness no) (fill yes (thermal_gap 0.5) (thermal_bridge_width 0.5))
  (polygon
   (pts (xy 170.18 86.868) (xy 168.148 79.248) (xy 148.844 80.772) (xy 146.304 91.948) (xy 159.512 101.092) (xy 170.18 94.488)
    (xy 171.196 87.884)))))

